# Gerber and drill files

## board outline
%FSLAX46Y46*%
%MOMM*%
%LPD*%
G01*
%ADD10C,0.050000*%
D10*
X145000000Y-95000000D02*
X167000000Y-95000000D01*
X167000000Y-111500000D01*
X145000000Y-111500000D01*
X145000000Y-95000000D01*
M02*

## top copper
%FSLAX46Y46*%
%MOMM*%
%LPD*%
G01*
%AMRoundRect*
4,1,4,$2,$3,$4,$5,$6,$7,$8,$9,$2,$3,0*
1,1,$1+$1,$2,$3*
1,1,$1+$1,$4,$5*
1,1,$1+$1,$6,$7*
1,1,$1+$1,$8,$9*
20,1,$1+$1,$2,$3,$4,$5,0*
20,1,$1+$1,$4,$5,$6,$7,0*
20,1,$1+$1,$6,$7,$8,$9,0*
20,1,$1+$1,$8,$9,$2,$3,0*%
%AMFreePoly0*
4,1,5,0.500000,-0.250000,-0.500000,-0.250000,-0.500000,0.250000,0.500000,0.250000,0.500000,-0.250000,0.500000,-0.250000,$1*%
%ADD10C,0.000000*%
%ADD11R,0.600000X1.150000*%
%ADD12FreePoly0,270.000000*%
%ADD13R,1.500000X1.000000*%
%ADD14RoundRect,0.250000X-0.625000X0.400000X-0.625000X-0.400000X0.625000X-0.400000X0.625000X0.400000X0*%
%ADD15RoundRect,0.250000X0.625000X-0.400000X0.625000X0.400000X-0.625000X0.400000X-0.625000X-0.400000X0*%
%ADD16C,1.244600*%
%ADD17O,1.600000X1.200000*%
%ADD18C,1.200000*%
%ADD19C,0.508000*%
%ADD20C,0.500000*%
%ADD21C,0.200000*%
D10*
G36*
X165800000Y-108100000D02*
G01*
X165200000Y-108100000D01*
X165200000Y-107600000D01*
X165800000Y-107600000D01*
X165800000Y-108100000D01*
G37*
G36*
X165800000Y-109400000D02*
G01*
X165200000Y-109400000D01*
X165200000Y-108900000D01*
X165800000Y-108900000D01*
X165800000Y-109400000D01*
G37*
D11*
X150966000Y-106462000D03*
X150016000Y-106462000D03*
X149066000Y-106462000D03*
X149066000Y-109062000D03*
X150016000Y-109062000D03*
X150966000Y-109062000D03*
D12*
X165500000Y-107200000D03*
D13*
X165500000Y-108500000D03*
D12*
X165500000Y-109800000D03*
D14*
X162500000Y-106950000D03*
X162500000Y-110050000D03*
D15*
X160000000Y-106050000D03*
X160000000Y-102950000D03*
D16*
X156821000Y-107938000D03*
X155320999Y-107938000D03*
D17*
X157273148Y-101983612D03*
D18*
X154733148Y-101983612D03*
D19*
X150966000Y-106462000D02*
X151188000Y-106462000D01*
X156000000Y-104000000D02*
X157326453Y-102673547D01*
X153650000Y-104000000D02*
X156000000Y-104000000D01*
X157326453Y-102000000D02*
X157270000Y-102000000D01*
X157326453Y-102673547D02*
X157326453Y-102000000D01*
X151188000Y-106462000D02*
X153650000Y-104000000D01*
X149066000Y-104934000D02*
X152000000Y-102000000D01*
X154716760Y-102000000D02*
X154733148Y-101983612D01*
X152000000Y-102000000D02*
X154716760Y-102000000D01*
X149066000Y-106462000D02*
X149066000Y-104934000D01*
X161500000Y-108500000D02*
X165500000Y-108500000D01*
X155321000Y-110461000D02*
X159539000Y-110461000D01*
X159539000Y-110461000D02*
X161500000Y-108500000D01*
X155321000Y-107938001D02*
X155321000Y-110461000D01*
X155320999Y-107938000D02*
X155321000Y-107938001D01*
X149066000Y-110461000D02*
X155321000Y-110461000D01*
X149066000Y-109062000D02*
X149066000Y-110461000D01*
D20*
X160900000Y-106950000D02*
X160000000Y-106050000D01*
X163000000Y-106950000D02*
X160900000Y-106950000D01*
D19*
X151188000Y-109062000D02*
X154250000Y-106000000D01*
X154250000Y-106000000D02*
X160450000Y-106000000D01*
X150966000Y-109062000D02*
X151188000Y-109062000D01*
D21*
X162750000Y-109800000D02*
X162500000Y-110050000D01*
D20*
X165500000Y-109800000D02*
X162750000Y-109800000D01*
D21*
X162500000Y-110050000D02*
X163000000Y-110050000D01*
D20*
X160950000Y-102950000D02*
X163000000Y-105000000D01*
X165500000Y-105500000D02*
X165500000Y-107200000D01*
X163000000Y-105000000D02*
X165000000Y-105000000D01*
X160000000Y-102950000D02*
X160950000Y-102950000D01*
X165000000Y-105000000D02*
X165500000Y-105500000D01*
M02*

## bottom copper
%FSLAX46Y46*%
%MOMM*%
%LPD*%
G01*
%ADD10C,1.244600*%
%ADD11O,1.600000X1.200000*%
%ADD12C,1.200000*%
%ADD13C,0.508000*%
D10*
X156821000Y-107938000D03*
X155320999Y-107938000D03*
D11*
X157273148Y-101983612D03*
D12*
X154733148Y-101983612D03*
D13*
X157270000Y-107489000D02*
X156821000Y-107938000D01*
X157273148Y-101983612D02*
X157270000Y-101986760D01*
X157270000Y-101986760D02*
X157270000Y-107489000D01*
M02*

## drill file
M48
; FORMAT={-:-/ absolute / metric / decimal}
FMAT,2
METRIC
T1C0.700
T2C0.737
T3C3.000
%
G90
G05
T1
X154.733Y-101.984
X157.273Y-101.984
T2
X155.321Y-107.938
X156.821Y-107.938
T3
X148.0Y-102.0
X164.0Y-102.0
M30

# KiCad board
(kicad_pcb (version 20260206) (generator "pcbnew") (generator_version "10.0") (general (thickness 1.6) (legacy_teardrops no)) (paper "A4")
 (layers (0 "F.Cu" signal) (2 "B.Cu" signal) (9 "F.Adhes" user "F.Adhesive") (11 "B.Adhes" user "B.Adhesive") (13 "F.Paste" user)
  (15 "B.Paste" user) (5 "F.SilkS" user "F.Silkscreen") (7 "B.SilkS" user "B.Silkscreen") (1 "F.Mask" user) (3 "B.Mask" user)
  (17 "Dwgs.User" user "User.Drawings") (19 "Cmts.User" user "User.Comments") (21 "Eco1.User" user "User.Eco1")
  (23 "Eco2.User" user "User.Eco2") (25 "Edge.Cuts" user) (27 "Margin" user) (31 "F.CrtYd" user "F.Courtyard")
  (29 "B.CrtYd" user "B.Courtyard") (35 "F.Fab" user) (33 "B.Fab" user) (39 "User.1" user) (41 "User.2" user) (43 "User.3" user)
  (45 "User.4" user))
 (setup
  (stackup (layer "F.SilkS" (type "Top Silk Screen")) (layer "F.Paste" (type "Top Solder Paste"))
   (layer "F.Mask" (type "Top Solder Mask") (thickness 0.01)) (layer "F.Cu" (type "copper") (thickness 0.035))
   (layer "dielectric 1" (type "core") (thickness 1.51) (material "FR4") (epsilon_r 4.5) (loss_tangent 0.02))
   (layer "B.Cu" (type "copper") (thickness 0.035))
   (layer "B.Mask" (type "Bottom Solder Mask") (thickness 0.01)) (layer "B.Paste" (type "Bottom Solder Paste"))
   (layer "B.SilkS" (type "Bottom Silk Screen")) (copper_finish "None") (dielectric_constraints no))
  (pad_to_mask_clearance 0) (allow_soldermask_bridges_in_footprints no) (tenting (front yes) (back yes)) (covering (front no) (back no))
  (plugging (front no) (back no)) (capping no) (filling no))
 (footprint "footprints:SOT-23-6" (layer "F.Cu") (at 150.016 107.762 -90)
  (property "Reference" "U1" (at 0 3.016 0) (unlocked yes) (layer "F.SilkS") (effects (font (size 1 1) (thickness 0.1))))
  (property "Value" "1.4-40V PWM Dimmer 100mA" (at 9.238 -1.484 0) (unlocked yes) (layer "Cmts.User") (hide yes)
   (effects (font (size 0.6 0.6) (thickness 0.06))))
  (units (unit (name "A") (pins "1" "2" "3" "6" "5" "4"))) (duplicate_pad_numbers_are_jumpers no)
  (pad "1" smd rect (at -1.3 -0.95 270) (size 1.15 0.6) (layers "F.Cu" "F.Mask" "F.Paste") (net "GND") (solder_mask_margin 0.1016)
   (solder_paste_margin 0) (thermal_bridge_angle 0))
  (pad "2" smd rect (at -1.3 0 270) (size 1.15 0.6) (layers "F.Cu" "F.Mask" "F.Paste") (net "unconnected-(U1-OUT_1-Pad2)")
   (solder_mask_margin 0.1016) (solder_paste_margin 0) (thermal_bridge_angle 0))
  (pad "3" smd rect (at -1.3 0.95 270) (size 1.15 0.6) (layers "F.Cu" "F.Mask" "F.Paste") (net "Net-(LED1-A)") (solder_mask_margin 0.1016)
   (solder_paste_margin 0) (thermal_bridge_angle 0))
  (pad "4" smd rect (at 1.3 0.95 270) (size 1.15 0.6) (layers "F.Cu" "F.Mask" "F.Paste") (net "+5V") (solder_mask_margin 0.1016)
   (solder_paste_margin 0) (thermal_bridge_angle 0))
  (pad "5" smd rect (at 1.3 0 270) (size 1.15 0.6) (layers "F.Cu" "F.Mask" "F.Paste") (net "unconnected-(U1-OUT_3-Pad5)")
   (solder_mask_margin 0.1016) (solder_paste_margin 0) (thermal_bridge_angle 0))
  (pad "6" smd rect (at 1.3 -0.95 270) (size 1.15 0.6) (layers "F.Cu" "F.Mask" "F.Paste") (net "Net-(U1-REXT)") (solder_mask_margin 0.1016)
   (solder_paste_margin 0) (thermal_bridge_angle 0)))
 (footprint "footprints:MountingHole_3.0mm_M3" (layer "F.Cu") (at 164 102)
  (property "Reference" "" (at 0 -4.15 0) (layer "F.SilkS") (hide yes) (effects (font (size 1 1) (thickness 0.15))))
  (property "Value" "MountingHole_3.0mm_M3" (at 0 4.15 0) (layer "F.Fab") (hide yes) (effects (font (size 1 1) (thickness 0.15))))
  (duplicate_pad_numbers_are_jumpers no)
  (pad "" np_thru_hole circle (at 0 0) (size 3 3) (drill 3) (layers "*.Cu" "*.Mask")))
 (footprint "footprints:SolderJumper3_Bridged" (layer "F.Cu") (at 165.5 108.5 -90)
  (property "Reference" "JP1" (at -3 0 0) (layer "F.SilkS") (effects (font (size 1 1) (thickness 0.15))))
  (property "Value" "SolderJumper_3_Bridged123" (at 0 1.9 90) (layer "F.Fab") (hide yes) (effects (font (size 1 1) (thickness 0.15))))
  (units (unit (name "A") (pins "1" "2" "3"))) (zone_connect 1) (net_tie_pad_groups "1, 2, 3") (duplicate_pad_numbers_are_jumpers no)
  (fp_poly (pts (xy -0.9 -0.3) (xy -0.4 -0.3) (xy -0.4 0.3) (xy -0.9 0.3)) (stroke (width 0) (type solid)) (fill yes) (layer "F.Cu"))
  (fp_poly (pts (xy 0.4 -0.3) (xy 0.9 -0.3) (xy 0.9 0.3) (xy 0.4 0.3)) (stroke (width 0) (type solid)) (fill yes) (layer "F.Cu"))
  (pad "1" smd custom (at -1.3 0 270) (size 1 0.5) (layers "F.Cu" "F.Mask") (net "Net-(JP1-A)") (zone_connect 2) (thermal_bridge_angle 45)
   (options (clearance outline) (anchor rect)) (primitives))
  (pad "2" smd rect (at 0 0 270) (size 1 1.5) (layers "F.Cu" "F.Mask") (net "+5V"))
  (pad "3" smd custom (at 1.3 0 270) (size 1 0.5) (layers "F.Cu" "F.Mask") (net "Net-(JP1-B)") (zone_connect 2) (thermal_bridge_angle 45)
   (options (clearance outline) (anchor rect)) (primitives)))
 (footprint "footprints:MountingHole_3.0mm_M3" (layer "F.Cu") (at 148 102)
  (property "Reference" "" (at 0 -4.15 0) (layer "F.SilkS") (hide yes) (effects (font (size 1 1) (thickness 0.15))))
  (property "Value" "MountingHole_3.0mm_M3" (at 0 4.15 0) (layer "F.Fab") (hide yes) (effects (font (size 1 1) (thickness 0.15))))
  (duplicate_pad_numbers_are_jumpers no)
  (pad "" np_thru_hole circle (at 0 0) (size 3 3) (drill 3) (layers "*.Cu" "*.Mask")))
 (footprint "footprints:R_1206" (layer "F.Cu") (at 162.5 108.5 -90)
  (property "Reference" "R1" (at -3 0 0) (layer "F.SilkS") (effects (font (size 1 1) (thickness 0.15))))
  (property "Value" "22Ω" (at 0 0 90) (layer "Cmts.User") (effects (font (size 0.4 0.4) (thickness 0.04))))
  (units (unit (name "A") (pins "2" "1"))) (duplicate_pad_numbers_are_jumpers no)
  (pad "1" smd roundrect (at -1.55 0 270) (size 1.3 1.75) (layers "F.Cu" "F.Mask" "F.Paste") (roundrect_rratio 0.192308)
   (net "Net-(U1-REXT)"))
  (pad "2" smd roundrect (at 1.55 0 270) (size 1.3 1.75) (layers "F.Cu" "F.Mask" "F.Paste") (roundrect_rratio 0.192308) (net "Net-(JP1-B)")))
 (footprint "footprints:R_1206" (layer "F.Cu") (at 160 104.5 90)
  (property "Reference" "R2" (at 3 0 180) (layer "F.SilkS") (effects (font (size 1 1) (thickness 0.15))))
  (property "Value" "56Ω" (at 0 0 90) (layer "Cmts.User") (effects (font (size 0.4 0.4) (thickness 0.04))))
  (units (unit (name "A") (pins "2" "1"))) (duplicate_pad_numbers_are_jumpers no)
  (pad "1" smd roundrect (at -1.55 0 90) (size 1.3 1.75) (layers "F.Cu" "F.Mask" "F.Paste") (roundrect_rratio 0.192308)
   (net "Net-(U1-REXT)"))
  (pad "2" smd roundrect (at 1.55 0 90) (size 1.3 1.75) (layers "F.Cu" "F.Mask" "F.Paste") (roundrect_rratio 0.192308) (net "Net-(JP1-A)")))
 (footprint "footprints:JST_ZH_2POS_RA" (layer "B.Cu") (at 156.821 107.938 180)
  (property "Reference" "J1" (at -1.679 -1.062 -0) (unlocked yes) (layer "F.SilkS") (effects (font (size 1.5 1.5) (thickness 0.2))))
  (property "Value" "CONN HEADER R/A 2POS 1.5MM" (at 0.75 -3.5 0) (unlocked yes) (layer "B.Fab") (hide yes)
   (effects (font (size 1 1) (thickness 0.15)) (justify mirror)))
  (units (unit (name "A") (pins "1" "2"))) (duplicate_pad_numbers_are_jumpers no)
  (pad "1" thru_hole circle (at 0 0 180) (size 1.2446 1.2446) (drill 0.7366) (layers "*.Cu" "*.Mask") (remove_unused_layers no) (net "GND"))
  (pad "2" thru_hole circle (at 1.500001 0 180) (size 1.2446 1.2446) (drill 0.7366) (layers "*.Cu" "*.Mask") (remove_unused_layers no)
   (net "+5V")))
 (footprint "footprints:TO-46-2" (layer "B.Cu") (at 157.273148 101.983612 180)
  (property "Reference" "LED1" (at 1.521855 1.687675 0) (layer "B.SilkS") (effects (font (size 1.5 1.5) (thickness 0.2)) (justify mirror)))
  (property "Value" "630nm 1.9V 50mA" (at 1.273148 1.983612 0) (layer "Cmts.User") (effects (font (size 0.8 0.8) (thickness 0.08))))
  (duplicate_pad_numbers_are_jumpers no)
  (pad "1" thru_hole oval (at 0 0 180) (size 1.6 1.2) (drill 0.7) (layers "*.Cu" "*.Mask") (remove_unused_layers no) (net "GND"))
  (pad "2" thru_hole circle (at 2.54 0 180) (size 1.2 1.2) (drill 0.7) (layers "*.Cu" "*.Mask") (remove_unused_layers no)
   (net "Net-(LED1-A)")))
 (gr_rect (start 145 95) (end 167 111.5) (stroke (width 0.05) (type default)) (fill no) (layer "Edge.Cuts"))
 (segment (start 150.966 106.462) (end 151.188 106.462) (width 0.508) (layer "F.Cu") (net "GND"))
 (segment (start 156 104) (end 157.326453 102.673547) (width 0.508) (layer "F.Cu") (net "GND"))
 (segment (start 153.65 104) (end 156 104) (width 0.508) (layer "F.Cu") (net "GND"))
 (segment (start 157.326453 102) (end 157.27 102) (width 0.508) (layer "F.Cu") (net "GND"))
 (segment (start 157.326453 102.673547) (end 157.326453 102) (width 0.508) (layer "F.Cu") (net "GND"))
 (segment (start 151.188 106.462) (end 153.65 104) (width 0.508) (layer "F.Cu") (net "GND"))
 (segment (start 157.27 107.489) (end 156.821 107.938) (width 0.508) (layer "B.Cu") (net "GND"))
 (segment (start 157.273148 101.983612) (end 157.27 101.98676) (width 0.508) (layer "B.Cu") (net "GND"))
 (segment (start 157.27 101.98676) (end 157.27 107.489) (width 0.508) (layer "B.Cu") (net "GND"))
 (segment (start 149.066 104.934) (end 152 102) (width 0.508) (layer "F.Cu") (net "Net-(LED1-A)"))
 (segment (start 154.71676 102) (end 154.733148 101.983612) (width 0.508) (layer "F.Cu") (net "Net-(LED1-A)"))
 (segment (start 152 102) (end 154.71676 102) (width 0.508) (layer "F.Cu") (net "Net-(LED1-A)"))
 (segment (start 149.066 106.462) (end 149.066 104.934) (width 0.508) (layer "F.Cu") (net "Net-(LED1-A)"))
 (segment (start 161.5 108.5) (end 165.5 108.5) (width 0.508) (layer "F.Cu") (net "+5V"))
 (segment (start 155.321 110.461) (end 159.539 110.461) (width 0.508) (layer "F.Cu") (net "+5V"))
 (segment (start 159.539 110.461) (end 161.5 108.5) (width 0.508) (layer "F.Cu") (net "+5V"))
 (segment (start 155.321 107.938001) (end 155.321 110.461) (width 0.508) (layer "F.Cu") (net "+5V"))
 (segment (start 155.320999 107.938) (end 155.321 107.938001) (width 0.508) (layer "F.Cu") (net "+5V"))
 (segment (start 149.066 110.461) (end 155.321 110.461) (width 0.508) (layer "F.Cu") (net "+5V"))
 (segment (start 149.066 109.062) (end 149.066 110.461) (width 0.508) (layer "F.Cu") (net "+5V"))
 (segment (start 160.9 106.95) (end 160 106.05) (width 0.5) (layer "F.Cu") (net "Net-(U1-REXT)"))
 (segment (start 163 106.95) (end 160.9 106.95) (width 0.5) (layer "F.Cu") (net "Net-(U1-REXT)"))
 (segment (start 151.188 109.062) (end 154.25 106) (width 0.508) (layer "F.Cu") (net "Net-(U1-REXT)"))
 (segment (start 154.25 106) (end 160.45 106) (width 0.508) (layer "F.Cu") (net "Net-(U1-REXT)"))
 (segment (start 150.966 109.062) (end 151.188 109.062) (width 0.508) (layer "F.Cu") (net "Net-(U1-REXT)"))
 (segment (start 162.75 109.8) (end 162.5 110.05) (width 0.2) (layer "F.Cu") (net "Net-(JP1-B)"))
 (segment (start 165.5 109.8) (end 162.75 109.8) (width 0.5) (layer "F.Cu") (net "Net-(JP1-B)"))
 (segment (start 162.5 110.05) (end 163 110.05) (width 0.2) (layer "F.Cu") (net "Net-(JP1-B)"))
 (segment (start 160.95 102.95) (end 163 105) (width 0.5) (layer "F.Cu") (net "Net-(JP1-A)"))
 (segment (start 165.5 105.5) (end 165.5 107.2) (width 0.5) (layer "F.Cu") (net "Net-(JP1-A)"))
 (segment (start 163 105) (end 165 105) (width 0.5) (layer "F.Cu") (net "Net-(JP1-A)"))
 (segment (start 160 102.95) (end 160.95 102.95) (width 0.5) (layer "F.Cu") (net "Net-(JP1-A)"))
 (segment (start 165 105) (end 165.5 105.5) (width 0.5) (layer "F.Cu") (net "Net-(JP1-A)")))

